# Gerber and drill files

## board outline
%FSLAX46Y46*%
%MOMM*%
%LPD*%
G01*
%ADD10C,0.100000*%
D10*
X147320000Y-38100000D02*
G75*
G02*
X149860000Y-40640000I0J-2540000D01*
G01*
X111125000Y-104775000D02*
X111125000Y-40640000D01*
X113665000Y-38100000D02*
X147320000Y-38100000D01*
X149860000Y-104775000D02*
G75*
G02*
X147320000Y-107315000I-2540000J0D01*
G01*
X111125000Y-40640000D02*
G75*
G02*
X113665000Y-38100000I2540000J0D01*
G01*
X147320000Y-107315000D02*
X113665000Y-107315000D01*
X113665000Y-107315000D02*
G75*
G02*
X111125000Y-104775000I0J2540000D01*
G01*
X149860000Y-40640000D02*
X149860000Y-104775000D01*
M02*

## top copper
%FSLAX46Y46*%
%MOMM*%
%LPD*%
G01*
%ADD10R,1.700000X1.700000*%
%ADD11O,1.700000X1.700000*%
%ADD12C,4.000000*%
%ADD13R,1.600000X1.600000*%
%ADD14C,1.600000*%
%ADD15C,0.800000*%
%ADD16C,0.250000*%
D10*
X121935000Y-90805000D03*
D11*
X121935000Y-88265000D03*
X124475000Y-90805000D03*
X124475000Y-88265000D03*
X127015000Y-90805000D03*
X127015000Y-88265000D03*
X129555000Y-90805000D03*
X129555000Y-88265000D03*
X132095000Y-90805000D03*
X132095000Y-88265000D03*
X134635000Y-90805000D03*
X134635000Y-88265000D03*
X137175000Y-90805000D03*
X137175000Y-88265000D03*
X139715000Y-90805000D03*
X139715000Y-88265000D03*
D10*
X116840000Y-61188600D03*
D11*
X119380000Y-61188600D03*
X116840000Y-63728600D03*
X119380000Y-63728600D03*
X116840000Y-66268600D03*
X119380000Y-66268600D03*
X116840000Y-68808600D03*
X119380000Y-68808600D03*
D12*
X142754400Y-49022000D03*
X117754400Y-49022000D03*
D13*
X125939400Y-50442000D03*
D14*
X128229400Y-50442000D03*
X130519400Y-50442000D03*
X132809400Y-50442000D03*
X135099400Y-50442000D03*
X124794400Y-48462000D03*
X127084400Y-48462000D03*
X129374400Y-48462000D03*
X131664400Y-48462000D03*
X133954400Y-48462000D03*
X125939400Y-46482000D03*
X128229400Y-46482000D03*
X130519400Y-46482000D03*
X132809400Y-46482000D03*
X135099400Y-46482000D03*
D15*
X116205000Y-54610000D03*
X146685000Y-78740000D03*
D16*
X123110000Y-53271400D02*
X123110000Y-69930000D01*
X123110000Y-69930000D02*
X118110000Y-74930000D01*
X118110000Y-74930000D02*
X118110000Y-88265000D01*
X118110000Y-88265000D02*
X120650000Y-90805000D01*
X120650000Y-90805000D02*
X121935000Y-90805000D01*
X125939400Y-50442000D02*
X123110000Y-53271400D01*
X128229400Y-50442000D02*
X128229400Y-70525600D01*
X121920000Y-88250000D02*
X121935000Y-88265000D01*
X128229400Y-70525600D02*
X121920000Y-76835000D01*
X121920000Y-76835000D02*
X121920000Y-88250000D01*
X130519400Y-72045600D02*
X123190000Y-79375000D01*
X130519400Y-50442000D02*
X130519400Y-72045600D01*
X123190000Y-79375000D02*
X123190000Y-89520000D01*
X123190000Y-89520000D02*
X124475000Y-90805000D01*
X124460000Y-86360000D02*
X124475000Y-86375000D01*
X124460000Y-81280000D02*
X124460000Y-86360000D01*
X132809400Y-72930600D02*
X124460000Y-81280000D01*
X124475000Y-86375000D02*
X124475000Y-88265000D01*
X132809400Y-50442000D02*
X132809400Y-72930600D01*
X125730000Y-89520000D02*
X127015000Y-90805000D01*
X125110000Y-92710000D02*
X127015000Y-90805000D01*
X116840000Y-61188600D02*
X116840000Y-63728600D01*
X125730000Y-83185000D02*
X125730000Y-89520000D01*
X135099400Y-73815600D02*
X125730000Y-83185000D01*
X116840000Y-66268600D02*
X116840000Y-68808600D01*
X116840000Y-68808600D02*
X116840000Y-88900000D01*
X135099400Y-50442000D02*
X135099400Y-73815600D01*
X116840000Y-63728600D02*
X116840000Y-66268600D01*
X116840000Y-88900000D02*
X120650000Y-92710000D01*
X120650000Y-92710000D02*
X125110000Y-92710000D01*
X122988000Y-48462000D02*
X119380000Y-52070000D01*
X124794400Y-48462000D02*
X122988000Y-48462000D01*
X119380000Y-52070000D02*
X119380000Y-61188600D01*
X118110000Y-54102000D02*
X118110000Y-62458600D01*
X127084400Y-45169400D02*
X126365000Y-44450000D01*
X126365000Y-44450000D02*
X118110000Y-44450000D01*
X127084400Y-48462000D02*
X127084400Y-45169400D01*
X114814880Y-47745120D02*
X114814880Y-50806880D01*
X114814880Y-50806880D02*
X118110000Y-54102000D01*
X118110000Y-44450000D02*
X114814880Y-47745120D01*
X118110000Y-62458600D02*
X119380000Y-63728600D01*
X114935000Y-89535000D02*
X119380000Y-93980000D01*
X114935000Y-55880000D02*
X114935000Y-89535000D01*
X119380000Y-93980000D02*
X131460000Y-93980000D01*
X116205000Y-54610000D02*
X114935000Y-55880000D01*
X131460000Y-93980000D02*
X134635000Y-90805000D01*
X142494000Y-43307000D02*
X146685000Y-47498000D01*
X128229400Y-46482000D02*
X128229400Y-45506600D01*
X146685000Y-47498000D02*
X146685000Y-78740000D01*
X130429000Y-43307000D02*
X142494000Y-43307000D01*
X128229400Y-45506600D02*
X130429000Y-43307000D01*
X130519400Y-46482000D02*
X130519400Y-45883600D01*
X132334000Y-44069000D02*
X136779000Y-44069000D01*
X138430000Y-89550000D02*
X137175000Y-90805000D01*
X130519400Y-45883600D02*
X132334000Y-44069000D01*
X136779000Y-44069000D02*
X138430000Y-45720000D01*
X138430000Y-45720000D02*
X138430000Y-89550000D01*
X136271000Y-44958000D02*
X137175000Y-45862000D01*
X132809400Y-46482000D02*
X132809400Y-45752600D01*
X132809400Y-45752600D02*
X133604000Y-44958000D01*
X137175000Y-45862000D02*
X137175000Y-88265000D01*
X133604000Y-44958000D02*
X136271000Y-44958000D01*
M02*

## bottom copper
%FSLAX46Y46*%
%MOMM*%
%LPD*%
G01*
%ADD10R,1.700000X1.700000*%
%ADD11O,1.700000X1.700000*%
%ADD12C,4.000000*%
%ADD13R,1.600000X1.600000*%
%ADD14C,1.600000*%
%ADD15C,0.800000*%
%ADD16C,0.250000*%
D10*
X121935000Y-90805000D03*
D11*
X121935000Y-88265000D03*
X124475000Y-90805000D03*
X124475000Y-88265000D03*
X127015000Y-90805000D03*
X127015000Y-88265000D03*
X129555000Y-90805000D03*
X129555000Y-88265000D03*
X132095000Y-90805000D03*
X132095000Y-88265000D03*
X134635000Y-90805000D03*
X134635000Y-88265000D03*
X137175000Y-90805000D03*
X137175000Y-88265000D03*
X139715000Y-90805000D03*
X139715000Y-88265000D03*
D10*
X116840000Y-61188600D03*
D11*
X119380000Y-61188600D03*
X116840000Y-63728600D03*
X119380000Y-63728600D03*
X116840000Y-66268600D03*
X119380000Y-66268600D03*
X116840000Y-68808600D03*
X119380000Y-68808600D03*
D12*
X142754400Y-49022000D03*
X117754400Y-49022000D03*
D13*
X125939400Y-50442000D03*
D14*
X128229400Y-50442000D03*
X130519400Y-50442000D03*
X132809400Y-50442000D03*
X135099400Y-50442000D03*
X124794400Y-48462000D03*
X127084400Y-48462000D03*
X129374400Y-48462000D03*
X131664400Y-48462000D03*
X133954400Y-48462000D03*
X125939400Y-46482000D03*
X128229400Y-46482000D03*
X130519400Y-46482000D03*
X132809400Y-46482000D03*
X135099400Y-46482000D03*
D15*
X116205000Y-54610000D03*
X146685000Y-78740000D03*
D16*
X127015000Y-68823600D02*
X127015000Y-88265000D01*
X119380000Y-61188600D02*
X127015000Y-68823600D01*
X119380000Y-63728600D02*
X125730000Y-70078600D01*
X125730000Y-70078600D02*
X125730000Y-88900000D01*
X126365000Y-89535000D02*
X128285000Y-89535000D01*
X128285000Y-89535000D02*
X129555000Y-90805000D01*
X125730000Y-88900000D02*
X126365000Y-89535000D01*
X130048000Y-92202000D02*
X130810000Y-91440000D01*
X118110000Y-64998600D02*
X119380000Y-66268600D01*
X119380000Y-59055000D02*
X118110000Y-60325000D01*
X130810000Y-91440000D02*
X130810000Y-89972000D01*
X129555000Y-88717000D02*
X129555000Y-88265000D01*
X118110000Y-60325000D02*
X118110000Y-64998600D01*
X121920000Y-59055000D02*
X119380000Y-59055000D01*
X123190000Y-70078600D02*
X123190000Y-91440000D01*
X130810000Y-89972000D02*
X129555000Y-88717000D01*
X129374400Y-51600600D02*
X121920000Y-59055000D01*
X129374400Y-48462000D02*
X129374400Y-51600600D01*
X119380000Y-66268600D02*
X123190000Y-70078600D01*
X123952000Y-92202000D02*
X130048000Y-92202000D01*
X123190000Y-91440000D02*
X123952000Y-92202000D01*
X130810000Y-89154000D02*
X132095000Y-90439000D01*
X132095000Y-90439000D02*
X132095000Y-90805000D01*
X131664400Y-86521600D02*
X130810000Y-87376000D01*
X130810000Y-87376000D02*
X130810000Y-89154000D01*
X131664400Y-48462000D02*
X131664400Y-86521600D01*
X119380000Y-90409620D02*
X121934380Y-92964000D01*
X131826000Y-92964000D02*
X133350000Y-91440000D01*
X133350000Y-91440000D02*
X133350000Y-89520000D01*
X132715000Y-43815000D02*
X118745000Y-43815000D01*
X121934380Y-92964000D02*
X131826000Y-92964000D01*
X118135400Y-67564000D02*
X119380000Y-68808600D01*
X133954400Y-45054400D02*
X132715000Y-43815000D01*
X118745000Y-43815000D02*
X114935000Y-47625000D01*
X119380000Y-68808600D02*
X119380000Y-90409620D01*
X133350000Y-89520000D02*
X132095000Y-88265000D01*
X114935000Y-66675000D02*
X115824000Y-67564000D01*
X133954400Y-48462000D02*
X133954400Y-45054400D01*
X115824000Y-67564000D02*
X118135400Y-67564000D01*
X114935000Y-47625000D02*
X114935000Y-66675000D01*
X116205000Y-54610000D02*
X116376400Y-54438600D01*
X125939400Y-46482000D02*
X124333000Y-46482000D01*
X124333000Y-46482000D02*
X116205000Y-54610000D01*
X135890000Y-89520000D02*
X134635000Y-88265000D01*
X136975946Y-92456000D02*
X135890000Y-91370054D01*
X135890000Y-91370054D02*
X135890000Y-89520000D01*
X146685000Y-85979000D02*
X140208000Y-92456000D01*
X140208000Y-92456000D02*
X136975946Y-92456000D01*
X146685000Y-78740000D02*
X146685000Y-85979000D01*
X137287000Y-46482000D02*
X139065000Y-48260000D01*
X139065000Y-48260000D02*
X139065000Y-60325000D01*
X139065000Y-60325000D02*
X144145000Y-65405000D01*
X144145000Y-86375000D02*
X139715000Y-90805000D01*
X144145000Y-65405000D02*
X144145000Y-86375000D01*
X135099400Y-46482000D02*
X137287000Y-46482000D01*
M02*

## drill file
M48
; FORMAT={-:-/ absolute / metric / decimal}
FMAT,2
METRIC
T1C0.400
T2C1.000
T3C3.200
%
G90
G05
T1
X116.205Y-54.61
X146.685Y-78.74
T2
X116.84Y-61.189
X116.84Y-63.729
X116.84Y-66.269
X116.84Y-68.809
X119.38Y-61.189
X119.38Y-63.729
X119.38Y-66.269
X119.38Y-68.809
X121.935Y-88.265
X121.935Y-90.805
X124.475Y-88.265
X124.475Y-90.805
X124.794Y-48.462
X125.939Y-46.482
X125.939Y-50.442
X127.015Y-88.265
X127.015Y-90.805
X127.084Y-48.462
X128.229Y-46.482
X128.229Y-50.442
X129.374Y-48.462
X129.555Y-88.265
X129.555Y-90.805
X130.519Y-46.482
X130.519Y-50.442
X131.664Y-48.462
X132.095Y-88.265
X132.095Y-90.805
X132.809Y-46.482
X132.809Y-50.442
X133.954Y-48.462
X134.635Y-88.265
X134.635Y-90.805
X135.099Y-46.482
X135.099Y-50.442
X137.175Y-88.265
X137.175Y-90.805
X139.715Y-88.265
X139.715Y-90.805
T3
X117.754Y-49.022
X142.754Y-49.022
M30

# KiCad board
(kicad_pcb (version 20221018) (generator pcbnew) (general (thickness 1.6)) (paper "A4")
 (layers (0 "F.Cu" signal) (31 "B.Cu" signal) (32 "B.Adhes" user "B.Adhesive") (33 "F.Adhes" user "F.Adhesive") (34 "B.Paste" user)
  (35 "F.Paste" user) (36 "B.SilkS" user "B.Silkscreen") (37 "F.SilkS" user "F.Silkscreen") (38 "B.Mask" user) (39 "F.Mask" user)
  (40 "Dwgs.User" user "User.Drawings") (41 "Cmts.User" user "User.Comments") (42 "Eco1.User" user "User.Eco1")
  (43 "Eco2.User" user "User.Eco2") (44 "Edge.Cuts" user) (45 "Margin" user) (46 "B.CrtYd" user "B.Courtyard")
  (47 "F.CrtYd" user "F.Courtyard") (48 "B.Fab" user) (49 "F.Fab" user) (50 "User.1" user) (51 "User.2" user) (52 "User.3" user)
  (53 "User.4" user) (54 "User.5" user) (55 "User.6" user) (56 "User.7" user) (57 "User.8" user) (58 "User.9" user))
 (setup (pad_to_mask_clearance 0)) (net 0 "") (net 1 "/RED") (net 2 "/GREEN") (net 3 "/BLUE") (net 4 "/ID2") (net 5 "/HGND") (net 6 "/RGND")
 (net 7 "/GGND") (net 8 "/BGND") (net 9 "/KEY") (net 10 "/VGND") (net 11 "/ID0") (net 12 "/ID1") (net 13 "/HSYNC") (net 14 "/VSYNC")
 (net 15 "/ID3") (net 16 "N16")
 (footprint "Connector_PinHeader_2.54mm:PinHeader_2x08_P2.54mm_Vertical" (layer "F.Cu") (at 121.935 90.805 90)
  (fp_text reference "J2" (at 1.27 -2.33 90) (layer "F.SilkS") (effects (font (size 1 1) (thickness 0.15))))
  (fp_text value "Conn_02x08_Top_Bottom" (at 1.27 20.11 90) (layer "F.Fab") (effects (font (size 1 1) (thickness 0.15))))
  (pad "1" thru_hole rect (at 0 0 90) (size 1.7 1.7) (drill 1) (layers "*.Cu" "*.Mask") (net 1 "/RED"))
  (pad "2" thru_hole oval (at 2.54 0 90) (size 1.7 1.7) (drill 1) (layers "*.Cu" "*.Mask") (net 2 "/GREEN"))
  (pad "3" thru_hole oval (at 0 2.54 90) (size 1.7 1.7) (drill 1) (layers "*.Cu" "*.Mask") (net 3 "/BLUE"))
  (pad "4" thru_hole oval (at 2.54 2.54 90) (size 1.7 1.7) (drill 1) (layers "*.Cu" "*.Mask") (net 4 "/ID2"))
  (pad "5" thru_hole oval (at 0 5.08 90) (size 1.7 1.7) (drill 1) (layers "*.Cu" "*.Mask") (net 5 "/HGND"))
  (pad "6" thru_hole oval (at 2.54 5.08 90) (size 1.7 1.7) (drill 1) (layers "*.Cu" "*.Mask") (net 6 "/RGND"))
  (pad "7" thru_hole oval (at 0 7.62 90) (size 1.7 1.7) (drill 1) (layers "*.Cu" "*.Mask") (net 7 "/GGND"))
  (pad "8" thru_hole oval (at 2.54 7.62 90) (size 1.7 1.7) (drill 1) (layers "*.Cu" "*.Mask") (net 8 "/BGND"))
  (pad "9" thru_hole oval (at 0 10.16 90) (size 1.7 1.7) (drill 1) (layers "*.Cu" "*.Mask") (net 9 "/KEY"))
  (pad "10" thru_hole oval (at 2.54 10.16 90) (size 1.7 1.7) (drill 1) (layers "*.Cu" "*.Mask") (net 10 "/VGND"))
  (pad "11" thru_hole oval (at 0 12.7 90) (size 1.7 1.7) (drill 1) (layers "*.Cu" "*.Mask") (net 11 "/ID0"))
  (pad "12" thru_hole oval (at 2.54 12.7 90) (size 1.7 1.7) (drill 1) (layers "*.Cu" "*.Mask") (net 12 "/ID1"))
  (pad "13" thru_hole oval (at 0 15.24 90) (size 1.7 1.7) (drill 1) (layers "*.Cu" "*.Mask") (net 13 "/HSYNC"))
  (pad "14" thru_hole oval (at 2.54 15.24 90) (size 1.7 1.7) (drill 1) (layers "*.Cu" "*.Mask") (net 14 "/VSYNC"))
  (pad "15" thru_hole oval (at 0 17.78 90) (size 1.7 1.7) (drill 1) (layers "*.Cu" "*.Mask") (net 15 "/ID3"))
  (pad "16" thru_hole oval (at 2.54 17.78 90) (size 1.7 1.7) (drill 1) (layers "*.Cu" "*.Mask") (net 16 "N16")))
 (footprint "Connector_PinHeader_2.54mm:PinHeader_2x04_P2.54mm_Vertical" (layer "F.Cu") (at 116.84 61.1886)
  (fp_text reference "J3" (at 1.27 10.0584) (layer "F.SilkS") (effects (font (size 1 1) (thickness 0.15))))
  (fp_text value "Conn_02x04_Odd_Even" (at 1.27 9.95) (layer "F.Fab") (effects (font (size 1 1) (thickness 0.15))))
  (pad "1" thru_hole rect (at 0 0) (size 1.7 1.7) (drill 1) (layers "*.Cu" "*.Mask") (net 5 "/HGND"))
  (pad "2" thru_hole oval (at 2.54 0) (size 1.7 1.7) (drill 1) (layers "*.Cu" "*.Mask") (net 6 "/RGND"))
  (pad "3" thru_hole oval (at 0 2.54) (size 1.7 1.7) (drill 1) (layers "*.Cu" "*.Mask") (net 5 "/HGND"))
  (pad "4" thru_hole oval (at 2.54 2.54) (size 1.7 1.7) (drill 1) (layers "*.Cu" "*.Mask") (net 7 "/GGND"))
  (pad "5" thru_hole oval (at 0 5.08) (size 1.7 1.7) (drill 1) (layers "*.Cu" "*.Mask") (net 5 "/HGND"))
  (pad "6" thru_hole oval (at 2.54 5.08) (size 1.7 1.7) (drill 1) (layers "*.Cu" "*.Mask") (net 8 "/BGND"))
  (pad "7" thru_hole oval (at 0 7.62) (size 1.7 1.7) (drill 1) (layers "*.Cu" "*.Mask") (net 5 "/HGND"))
  (pad "8" thru_hole oval (at 2.54 7.62) (size 1.7 1.7) (drill 1) (layers "*.Cu" "*.Mask") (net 10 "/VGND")))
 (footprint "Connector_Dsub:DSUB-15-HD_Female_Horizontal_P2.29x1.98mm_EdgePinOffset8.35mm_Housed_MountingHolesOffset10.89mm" (layer "F.Cu")
  (at 125.9394 50.442 180)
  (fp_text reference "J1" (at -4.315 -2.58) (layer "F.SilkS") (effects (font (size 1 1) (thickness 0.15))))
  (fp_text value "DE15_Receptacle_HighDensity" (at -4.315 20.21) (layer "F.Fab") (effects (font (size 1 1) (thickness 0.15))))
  (pad "0" thru_hole circle (at -16.815 1.42 180) (size 4 4) (drill 3.2) (layers "*.Cu" "*.Mask"))
  (pad "0" thru_hole circle (at 8.185 1.42 180) (size 4 4) (drill 3.2) (layers "*.Cu" "*.Mask"))
  (pad "1" thru_hole rect (at 0 0 180) (size 1.6 1.6) (drill 1) (layers "*.Cu" "*.Mask") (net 1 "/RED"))
  (pad "2" thru_hole circle (at -2.29 0 180) (size 1.6 1.6) (drill 1) (layers "*.Cu" "*.Mask") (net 2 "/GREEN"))
  (pad "3" thru_hole circle (at -4.58 0 180) (size 1.6 1.6) (drill 1) (layers "*.Cu" "*.Mask") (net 3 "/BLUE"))
  (pad "4" thru_hole circle (at -6.87 0 180) (size 1.6 1.6) (drill 1) (layers "*.Cu" "*.Mask") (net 4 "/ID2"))
  (pad "5" thru_hole circle (at -9.16 0 180) (size 1.6 1.6) (drill 1) (layers "*.Cu" "*.Mask") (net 5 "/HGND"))
  (pad "6" thru_hole circle (at 1.145 1.98 180) (size 1.6 1.6) (drill 1) (layers "*.Cu" "*.Mask") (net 6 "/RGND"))
  (pad "7" thru_hole circle (at -1.145 1.98 180) (size 1.6 1.6) (drill 1) (layers "*.Cu" "*.Mask") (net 7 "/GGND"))
  (pad "8" thru_hole circle (at -3.435 1.98 180) (size 1.6 1.6) (drill 1) (layers "*.Cu" "*.Mask") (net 8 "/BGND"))
  (pad "9" thru_hole circle (at -5.725 1.98 180) (size 1.6 1.6) (drill 1) (layers "*.Cu" "*.Mask") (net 9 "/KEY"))
  (pad "10" thru_hole circle (at -8.015 1.98 180) (size 1.6 1.6) (drill 1) (layers "*.Cu" "*.Mask") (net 10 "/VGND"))
  (pad "11" thru_hole circle (at 0 3.96 180) (size 1.6 1.6) (drill 1) (layers "*.Cu" "*.Mask") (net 11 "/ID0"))
  (pad "12" thru_hole circle (at -2.29 3.96 180) (size 1.6 1.6) (drill 1) (layers "*.Cu" "*.Mask") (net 12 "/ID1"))
  (pad "13" thru_hole circle (at -4.58 3.96 180) (size 1.6 1.6) (drill 1) (layers "*.Cu" "*.Mask") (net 13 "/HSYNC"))
  (pad "14" thru_hole circle (at -6.87 3.96 180) (size 1.6 1.6) (drill 1) (layers "*.Cu" "*.Mask") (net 14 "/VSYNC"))
  (pad "15" thru_hole circle (at -9.16 3.96 180) (size 1.6 1.6) (drill 1) (layers "*.Cu" "*.Mask") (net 15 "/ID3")))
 (gr_arc (start 147.32 38.1) (mid 149.116051 38.843949) (end 149.86 40.64) (stroke (width 0.1) (type default)) (layer "Edge.Cuts"))
 (gr_line (start 111.125 104.775) (end 111.125 40.64) (stroke (width 0.1) (type default)) (layer "Edge.Cuts"))
 (gr_line (start 113.665 38.1) (end 147.32 38.1) (stroke (width 0.1) (type default)) (layer "Edge.Cuts"))
 (gr_arc (start 149.86 104.775) (mid 149.116051 106.571051) (end 147.32 107.315) (stroke (width 0.1) (type default)) (layer "Edge.Cuts"))
 (gr_arc (start 111.125 40.64) (mid 111.868949 38.843949) (end 113.665 38.1) (stroke (width 0.1) (type default)) (layer "Edge.Cuts"))
 (gr_line (start 147.32 107.315) (end 113.665 107.315) (stroke (width 0.1) (type default)) (layer "Edge.Cuts"))
 (gr_arc (start 113.665 107.315) (mid 111.868949 106.571051) (end 111.125 104.775) (stroke (width 0.1) (type default)) (layer "Edge.Cuts"))
 (gr_line (start 149.86 40.64) (end 149.86 104.775) (stroke (width 0.1) (type default)) (layer "Edge.Cuts"))
 (segment (start 123.11 53.2714) (end 123.11 69.93) (width 0.25) (layer "F.Cu") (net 1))
 (segment (start 123.11 69.93) (end 118.11 74.93) (width 0.25) (layer "F.Cu") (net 1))
 (segment (start 118.11 74.93) (end 118.11 88.265) (width 0.25) (layer "F.Cu") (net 1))
 (segment (start 118.11 88.265) (end 120.65 90.805) (width 0.25) (layer "F.Cu") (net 1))
 (segment (start 120.65 90.805) (end 121.935 90.805) (width 0.25) (layer "F.Cu") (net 1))
 (segment (start 125.9394 50.442) (end 123.11 53.2714) (width 0.25) (layer "F.Cu") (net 1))
 (segment (start 128.2294 50.442) (end 128.2294 70.5256) (width 0.25) (layer "F.Cu") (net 2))
 (segment (start 121.92 88.25) (end 121.935 88.265) (width 0.25) (layer "F.Cu") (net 2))
 (segment (start 128.2294 70.5256) (end 121.92 76.835) (width 0.25) (layer "F.Cu") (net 2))
 (segment (start 121.92 76.835) (end 121.92 88.25) (width 0.25) (layer "F.Cu") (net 2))
 (segment (start 130.5194 72.0456) (end 123.19 79.375) (width 0.25) (layer "F.Cu") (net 3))
 (segment (start 130.5194 50.442) (end 130.5194 72.0456) (width 0.25) (layer "F.Cu") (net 3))
 (segment (start 123.19 79.375) (end 123.19 89.52) (width 0.25) (layer "F.Cu") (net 3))
 (segment (start 123.19 89.52) (end 124.475 90.805) (width 0.25) (layer "F.Cu") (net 3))
 (segment (start 124.46 86.36) (end 124.475 86.375) (width 0.25) (layer "F.Cu") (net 4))
 (segment (start 124.46 81.28) (end 124.46 86.36) (width 0.25) (layer "F.Cu") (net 4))
 (segment (start 132.8094 72.9306) (end 124.46 81.28) (width 0.25) (layer "F.Cu") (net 4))
 (segment (start 124.475 86.375) (end 124.475 88.265) (width 0.25) (layer "F.Cu") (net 4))
 (segment (start 132.8094 50.442) (end 132.8094 72.9306) (width 0.25) (layer "F.Cu") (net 4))
 (segment (start 125.73 89.52) (end 127.015 90.805) (width 0.25) (layer "F.Cu") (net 5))
 (segment (start 125.11 92.71) (end 127.015 90.805) (width 0.25) (layer "F.Cu") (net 5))
 (segment (start 116.84 61.1886) (end 116.84 63.7286) (width 0.25) (layer "F.Cu") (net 5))
 (segment (start 125.73 83.185) (end 125.73 89.52) (width 0.25) (layer "F.Cu") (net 5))
 (segment (start 135.0994 73.8156) (end 125.73 83.185) (width 0.25) (layer "F.Cu") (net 5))
 (segment (start 116.84 66.2686) (end 116.84 68.8086) (width 0.25) (layer "F.Cu") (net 5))
 (segment (start 116.84 68.8086) (end 116.84 88.9) (width 0.25) (layer "F.Cu") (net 5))
 (segment (start 135.0994 50.442) (end 135.0994 73.8156) (width 0.25) (layer "F.Cu") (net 5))
 (segment (start 116.84 63.7286) (end 116.84 66.2686) (width 0.25) (layer "F.Cu") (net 5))
 (segment (start 116.84 88.9) (end 120.65 92.71) (width 0.25) (layer "F.Cu") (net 5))
 (segment (start 120.65 92.71) (end 125.11 92.71) (width 0.25) (layer "F.Cu") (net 5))
 (segment (start 122.988 48.462) (end 119.38 52.07) (width 0.25) (layer "F.Cu") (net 6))
 (segment (start 124.7944 48.462) (end 122.988 48.462) (width 0.25) (layer "F.Cu") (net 6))
 (segment (start 119.38 52.07) (end 119.38 61.1886) (width 0.25) (layer "F.Cu") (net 6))
 (segment (start 127.015 68.8236) (end 127.015 88.265) (width 0.25) (layer "B.Cu") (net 6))
 (segment (start 119.38 61.1886) (end 127.015 68.8236) (width 0.25) (layer "B.Cu") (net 6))
 (segment (start 118.11 54.102) (end 118.11 62.4586) (width 0.25) (layer "F.Cu") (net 7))
 (segment (start 127.0844 45.1694) (end 126.365 44.45) (width 0.25) (layer "F.Cu") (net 7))
 (segment (start 126.365 44.45) (end 118.11 44.45) (width 0.25) (layer "F.Cu") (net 7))
 (segment (start 127.0844 48.462) (end 127.0844 45.1694) (width 0.25) (layer "F.Cu") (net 7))
 (segment (start 114.81488 47.74512) (end 114.81488 50.80688) (width 0.25) (layer "F.Cu") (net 7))
 (segment (start 114.81488 50.80688) (end 118.11 54.102) (width 0.25) (layer "F.Cu") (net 7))
 (segment (start 118.11 44.45) (end 114.81488 47.74512) (width 0.25) (layer "F.Cu") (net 7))
 (segment (start 118.11 62.4586) (end 119.38 63.7286) (width 0.25) (layer "F.Cu") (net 7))
 (segment (start 119.38 63.7286) (end 125.73 70.0786) (width 0.25) (layer "B.Cu") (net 7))
 (segment (start 125.73 70.0786) (end 125.73 88.9) (width 0.25) (layer "B.Cu") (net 7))
 (segment (start 126.365 89.535) (end 128.285 89.535) (width 0.25) (layer "B.Cu") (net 7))
 (segment (start 128.285 89.535) (end 129.555 90.805) (width 0.25) (layer "B.Cu") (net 7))
 (segment (start 125.73 88.9) (end 126.365 89.535) (width 0.25) (layer "B.Cu") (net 7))
 (segment (start 130.048 92.202) (end 130.81 91.44) (width 0.25) (layer "B.Cu") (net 8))
 (segment (start 118.11 64.9986) (end 119.38 66.2686) (width 0.25) (layer "B.Cu") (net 8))
 (segment (start 119.38 59.055) (end 118.11 60.325) (width 0.25) (layer "B.Cu") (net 8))
 (segment (start 130.81 91.44) (end 130.81 89.972) (width 0.25) (layer "B.Cu") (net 8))
 (segment (start 129.555 88.717) (end 129.555 88.265) (width 0.25) (layer "B.Cu") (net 8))
 (segment (start 118.11 60.325) (end 118.11 64.9986) (width 0.25) (layer "B.Cu") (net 8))
 (segment (start 121.92 59.055) (end 119.38 59.055) (width 0.25) (layer "B.Cu") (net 8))
 (segment (start 123.19 70.0786) (end 123.19 91.44) (width 0.25) (layer "B.Cu") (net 8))
 (segment (start 130.81 89.972) (end 129.555 88.717) (width 0.25) (layer "B.Cu") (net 8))
 (segment (start 129.3744 51.6006) (end 121.92 59.055) (width 0.25) (layer "B.Cu") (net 8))
 (segment (start 129.3744 48.462) (end 129.3744 51.6006) (width 0.25) (layer "B.Cu") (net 8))
 (segment (start 119.38 66.2686) (end 123.19 70.0786) (width 0.25) (layer "B.Cu") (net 8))
 (segment (start 123.952 92.202) (end 130.048 92.202) (width 0.25) (layer "B.Cu") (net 8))
 (segment (start 123.19 91.44) (end 123.952 92.202) (width 0.25) (layer "B.Cu") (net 8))
 (segment (start 130.81 89.154) (end 132.095 90.439) (width 0.25) (layer "B.Cu") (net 9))
 (segment (start 132.095 90.439) (end 132.095 90.805) (width 0.25) (layer "B.Cu") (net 9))
 (segment (start 131.6644 86.5216) (end 130.81 87.376) (width 0.25) (layer "B.Cu") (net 9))
 (segment (start 130.81 87.376) (end 130.81 89.154) (width 0.25) (layer "B.Cu") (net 9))
 (segment (start 131.6644 48.462) (end 131.6644 86.5216) (width 0.25) (layer "B.Cu") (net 9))
 (segment (start 119.38 90.40962) (end 121.93438 92.964) (width 0.25) (layer "B.Cu") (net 10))
 (segment (start 131.826 92.964) (end 133.35 91.44) (width 0.25) (layer "B.Cu") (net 10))
 (segment (start 133.35 91.44) (end 133.35 89.52) (width 0.25) (layer "B.Cu") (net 10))
 (segment (start 132.715 43.815) (end 118.745 43.815) (width 0.25) (layer "B.Cu") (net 10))
 (segment (start 121.93438 92.964) (end 131.826 92.964) (width 0.25) (layer "B.Cu") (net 10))
 (segment (start 118.1354 67.564) (end 119.38 68.8086) (width 0.25) (layer "B.Cu") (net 10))
 (segment (start 133.9544 45.0544) (end 132.715 43.815) (width 0.25) (layer "B.Cu") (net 10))
 (segment (start 118.745 43.815) (end 114.935 47.625) (width 0.25) (layer "B.Cu") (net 10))
 (segment (start 119.38 68.8086) (end 119.38 90.40962) (width 0.25) (layer "B.Cu") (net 10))
 (segment (start 133.35 89.52) (end 132.095 88.265) (width 0.25) (layer "B.Cu") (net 10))
 (segment (start 114.935 66.675) (end 115.824 67.564) (width 0.25) (layer "B.Cu") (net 10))
 (segment (start 133.9544 48.462) (end 133.9544 45.0544) (width 0.25) (layer "B.Cu") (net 10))
 (segment (start 115.824 67.564) (end 118.1354 67.564) (width 0.25) (layer "B.Cu") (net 10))
 (segment (start 114.935 47.625) (end 114.935 66.675) (width 0.25) (layer "B.Cu") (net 10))
 (segment (start 114.935 89.535) (end 119.38 93.98) (width 0.25) (layer "F.Cu") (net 11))
 (segment (start 114.935 55.88) (end 114.935 89.535) (width 0.25) (layer "F.Cu") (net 11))
 (segment (start 119.38 93.98) (end 131.46 93.98) (width 0.25) (layer "F.Cu") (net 11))
 (segment (start 116.205 54.61) (end 114.935 55.88) (width 0.25) (layer "F.Cu") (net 11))
 (segment (start 131.46 93.98) (end 134.635 90.805) (width 0.25) (layer "F.Cu") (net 11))
 (via (at 116.205 54.61) (size 0.8) (drill 0.4) (layers "F.Cu" "B.Cu") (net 11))
 (segment (start 116.205 54.61) (end 116.3764 54.4386) (width 0.25) (layer "B.Cu") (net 11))
 (segment (start 125.9394 46.482) (end 124.333 46.482) (width 0.25) (layer "B.Cu") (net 11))
 (segment (start 124.333 46.482) (end 116.205 54.61) (width 0.25) (layer "B.Cu") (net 11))
 (segment (start 142.494 43.307) (end 146.685 47.498) (width 0.25) (layer "F.Cu") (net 12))
 (segment (start 128.2294 46.482) (end 128.2294 45.5066) (width 0.25) (layer "F.Cu") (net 12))
 (segment (start 146.685 47.498) (end 146.685 78.74) (width 0.25) (layer "F.Cu") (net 12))
 (segment (start 130.429 43.307) (end 142.494 43.307) (width 0.25) (layer "F.Cu") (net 12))
 (segment (start 128.2294 45.5066) (end 130.429 43.307) (width 0.25) (layer "F.Cu") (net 12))
 (via (at 146.685 78.74) (size 0.8) (drill 0.4) (layers "F.Cu" "B.Cu") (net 12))
 (segment (start 135.89 89.52) (end 134.635 88.265) (width 0.25) (layer "B.Cu") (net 12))
 (segment (start 136.975946 92.456) (end 135.89 91.370054) (width 0.25) (layer "B.Cu") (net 12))
 (segment (start 135.89 91.370054) (end 135.89 89.52) (width 0.25) (layer "B.Cu") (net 12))
 (segment (start 146.685 85.979) (end 140.208 92.456) (width 0.25) (layer "B.Cu") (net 12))
 (segment (start 140.208 92.456) (end 136.975946 92.456) (width 0.25) (layer "B.Cu") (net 12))
 (segment (start 146.685 78.74) (end 146.685 85.979) (width 0.25) (layer "B.Cu") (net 12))
 (segment (start 130.5194 46.482) (end 130.5194 45.8836) (width 0.25) (layer "F.Cu") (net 13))
 (segment (start 132.334 44.069) (end 136.779 44.069) (width 0.25) (layer "F.Cu") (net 13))
 (segment (start 138.43 89.55) (end 137.175 90.805) (width 0.25) (layer "F.Cu") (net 13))
 (segment (start 130.5194 45.8836) (end 132.334 44.069) (width 0.25) (layer "F.Cu") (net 13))
 (segment (start 136.779 44.069) (end 138.43 45.72) (width 0.25) (layer "F.Cu") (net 13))
 (segment (start 138.43 45.72) (end 138.43 89.55) (width 0.25) (layer "F.Cu") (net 13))
 (segment (start 136.271 44.958) (end 137.175 45.862) (width 0.25) (layer "F.Cu") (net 14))
 (segment (start 132.8094 46.482) (end 132.8094 45.7526) (width 0.25) (layer "F.Cu") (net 14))
 (segment (start 132.8094 45.7526) (end 133.604 44.958) (width 0.25) (layer "F.Cu") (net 14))
 (segment (start 137.175 45.862) (end 137.175 88.265) (width 0.25) (layer "F.Cu") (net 14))
 (segment (start 133.604 44.958) (end 136.271 44.958) (width 0.25) (layer "F.Cu") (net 14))
 (segment (start 137.287 46.482) (end 139.065 48.26) (width 0.25) (layer "B.Cu") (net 15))
 (segment (start 139.065 48.26) (end 139.065 60.325) (width 0.25) (layer "B.Cu") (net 15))
 (segment (start 139.065 60.325) (end 144.145 65.405) (width 0.25) (layer "B.Cu") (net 15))
 (segment (start 144.145 86.375) (end 139.715 90.805) (width 0.25) (layer "B.Cu") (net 15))
 (segment (start 144.145 65.405) (end 144.145 86.375) (width 0.25) (layer "B.Cu") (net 15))
 (segment (start 135.0994 46.482) (end 137.287 46.482) (width 0.25) (layer "B.Cu") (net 15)))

